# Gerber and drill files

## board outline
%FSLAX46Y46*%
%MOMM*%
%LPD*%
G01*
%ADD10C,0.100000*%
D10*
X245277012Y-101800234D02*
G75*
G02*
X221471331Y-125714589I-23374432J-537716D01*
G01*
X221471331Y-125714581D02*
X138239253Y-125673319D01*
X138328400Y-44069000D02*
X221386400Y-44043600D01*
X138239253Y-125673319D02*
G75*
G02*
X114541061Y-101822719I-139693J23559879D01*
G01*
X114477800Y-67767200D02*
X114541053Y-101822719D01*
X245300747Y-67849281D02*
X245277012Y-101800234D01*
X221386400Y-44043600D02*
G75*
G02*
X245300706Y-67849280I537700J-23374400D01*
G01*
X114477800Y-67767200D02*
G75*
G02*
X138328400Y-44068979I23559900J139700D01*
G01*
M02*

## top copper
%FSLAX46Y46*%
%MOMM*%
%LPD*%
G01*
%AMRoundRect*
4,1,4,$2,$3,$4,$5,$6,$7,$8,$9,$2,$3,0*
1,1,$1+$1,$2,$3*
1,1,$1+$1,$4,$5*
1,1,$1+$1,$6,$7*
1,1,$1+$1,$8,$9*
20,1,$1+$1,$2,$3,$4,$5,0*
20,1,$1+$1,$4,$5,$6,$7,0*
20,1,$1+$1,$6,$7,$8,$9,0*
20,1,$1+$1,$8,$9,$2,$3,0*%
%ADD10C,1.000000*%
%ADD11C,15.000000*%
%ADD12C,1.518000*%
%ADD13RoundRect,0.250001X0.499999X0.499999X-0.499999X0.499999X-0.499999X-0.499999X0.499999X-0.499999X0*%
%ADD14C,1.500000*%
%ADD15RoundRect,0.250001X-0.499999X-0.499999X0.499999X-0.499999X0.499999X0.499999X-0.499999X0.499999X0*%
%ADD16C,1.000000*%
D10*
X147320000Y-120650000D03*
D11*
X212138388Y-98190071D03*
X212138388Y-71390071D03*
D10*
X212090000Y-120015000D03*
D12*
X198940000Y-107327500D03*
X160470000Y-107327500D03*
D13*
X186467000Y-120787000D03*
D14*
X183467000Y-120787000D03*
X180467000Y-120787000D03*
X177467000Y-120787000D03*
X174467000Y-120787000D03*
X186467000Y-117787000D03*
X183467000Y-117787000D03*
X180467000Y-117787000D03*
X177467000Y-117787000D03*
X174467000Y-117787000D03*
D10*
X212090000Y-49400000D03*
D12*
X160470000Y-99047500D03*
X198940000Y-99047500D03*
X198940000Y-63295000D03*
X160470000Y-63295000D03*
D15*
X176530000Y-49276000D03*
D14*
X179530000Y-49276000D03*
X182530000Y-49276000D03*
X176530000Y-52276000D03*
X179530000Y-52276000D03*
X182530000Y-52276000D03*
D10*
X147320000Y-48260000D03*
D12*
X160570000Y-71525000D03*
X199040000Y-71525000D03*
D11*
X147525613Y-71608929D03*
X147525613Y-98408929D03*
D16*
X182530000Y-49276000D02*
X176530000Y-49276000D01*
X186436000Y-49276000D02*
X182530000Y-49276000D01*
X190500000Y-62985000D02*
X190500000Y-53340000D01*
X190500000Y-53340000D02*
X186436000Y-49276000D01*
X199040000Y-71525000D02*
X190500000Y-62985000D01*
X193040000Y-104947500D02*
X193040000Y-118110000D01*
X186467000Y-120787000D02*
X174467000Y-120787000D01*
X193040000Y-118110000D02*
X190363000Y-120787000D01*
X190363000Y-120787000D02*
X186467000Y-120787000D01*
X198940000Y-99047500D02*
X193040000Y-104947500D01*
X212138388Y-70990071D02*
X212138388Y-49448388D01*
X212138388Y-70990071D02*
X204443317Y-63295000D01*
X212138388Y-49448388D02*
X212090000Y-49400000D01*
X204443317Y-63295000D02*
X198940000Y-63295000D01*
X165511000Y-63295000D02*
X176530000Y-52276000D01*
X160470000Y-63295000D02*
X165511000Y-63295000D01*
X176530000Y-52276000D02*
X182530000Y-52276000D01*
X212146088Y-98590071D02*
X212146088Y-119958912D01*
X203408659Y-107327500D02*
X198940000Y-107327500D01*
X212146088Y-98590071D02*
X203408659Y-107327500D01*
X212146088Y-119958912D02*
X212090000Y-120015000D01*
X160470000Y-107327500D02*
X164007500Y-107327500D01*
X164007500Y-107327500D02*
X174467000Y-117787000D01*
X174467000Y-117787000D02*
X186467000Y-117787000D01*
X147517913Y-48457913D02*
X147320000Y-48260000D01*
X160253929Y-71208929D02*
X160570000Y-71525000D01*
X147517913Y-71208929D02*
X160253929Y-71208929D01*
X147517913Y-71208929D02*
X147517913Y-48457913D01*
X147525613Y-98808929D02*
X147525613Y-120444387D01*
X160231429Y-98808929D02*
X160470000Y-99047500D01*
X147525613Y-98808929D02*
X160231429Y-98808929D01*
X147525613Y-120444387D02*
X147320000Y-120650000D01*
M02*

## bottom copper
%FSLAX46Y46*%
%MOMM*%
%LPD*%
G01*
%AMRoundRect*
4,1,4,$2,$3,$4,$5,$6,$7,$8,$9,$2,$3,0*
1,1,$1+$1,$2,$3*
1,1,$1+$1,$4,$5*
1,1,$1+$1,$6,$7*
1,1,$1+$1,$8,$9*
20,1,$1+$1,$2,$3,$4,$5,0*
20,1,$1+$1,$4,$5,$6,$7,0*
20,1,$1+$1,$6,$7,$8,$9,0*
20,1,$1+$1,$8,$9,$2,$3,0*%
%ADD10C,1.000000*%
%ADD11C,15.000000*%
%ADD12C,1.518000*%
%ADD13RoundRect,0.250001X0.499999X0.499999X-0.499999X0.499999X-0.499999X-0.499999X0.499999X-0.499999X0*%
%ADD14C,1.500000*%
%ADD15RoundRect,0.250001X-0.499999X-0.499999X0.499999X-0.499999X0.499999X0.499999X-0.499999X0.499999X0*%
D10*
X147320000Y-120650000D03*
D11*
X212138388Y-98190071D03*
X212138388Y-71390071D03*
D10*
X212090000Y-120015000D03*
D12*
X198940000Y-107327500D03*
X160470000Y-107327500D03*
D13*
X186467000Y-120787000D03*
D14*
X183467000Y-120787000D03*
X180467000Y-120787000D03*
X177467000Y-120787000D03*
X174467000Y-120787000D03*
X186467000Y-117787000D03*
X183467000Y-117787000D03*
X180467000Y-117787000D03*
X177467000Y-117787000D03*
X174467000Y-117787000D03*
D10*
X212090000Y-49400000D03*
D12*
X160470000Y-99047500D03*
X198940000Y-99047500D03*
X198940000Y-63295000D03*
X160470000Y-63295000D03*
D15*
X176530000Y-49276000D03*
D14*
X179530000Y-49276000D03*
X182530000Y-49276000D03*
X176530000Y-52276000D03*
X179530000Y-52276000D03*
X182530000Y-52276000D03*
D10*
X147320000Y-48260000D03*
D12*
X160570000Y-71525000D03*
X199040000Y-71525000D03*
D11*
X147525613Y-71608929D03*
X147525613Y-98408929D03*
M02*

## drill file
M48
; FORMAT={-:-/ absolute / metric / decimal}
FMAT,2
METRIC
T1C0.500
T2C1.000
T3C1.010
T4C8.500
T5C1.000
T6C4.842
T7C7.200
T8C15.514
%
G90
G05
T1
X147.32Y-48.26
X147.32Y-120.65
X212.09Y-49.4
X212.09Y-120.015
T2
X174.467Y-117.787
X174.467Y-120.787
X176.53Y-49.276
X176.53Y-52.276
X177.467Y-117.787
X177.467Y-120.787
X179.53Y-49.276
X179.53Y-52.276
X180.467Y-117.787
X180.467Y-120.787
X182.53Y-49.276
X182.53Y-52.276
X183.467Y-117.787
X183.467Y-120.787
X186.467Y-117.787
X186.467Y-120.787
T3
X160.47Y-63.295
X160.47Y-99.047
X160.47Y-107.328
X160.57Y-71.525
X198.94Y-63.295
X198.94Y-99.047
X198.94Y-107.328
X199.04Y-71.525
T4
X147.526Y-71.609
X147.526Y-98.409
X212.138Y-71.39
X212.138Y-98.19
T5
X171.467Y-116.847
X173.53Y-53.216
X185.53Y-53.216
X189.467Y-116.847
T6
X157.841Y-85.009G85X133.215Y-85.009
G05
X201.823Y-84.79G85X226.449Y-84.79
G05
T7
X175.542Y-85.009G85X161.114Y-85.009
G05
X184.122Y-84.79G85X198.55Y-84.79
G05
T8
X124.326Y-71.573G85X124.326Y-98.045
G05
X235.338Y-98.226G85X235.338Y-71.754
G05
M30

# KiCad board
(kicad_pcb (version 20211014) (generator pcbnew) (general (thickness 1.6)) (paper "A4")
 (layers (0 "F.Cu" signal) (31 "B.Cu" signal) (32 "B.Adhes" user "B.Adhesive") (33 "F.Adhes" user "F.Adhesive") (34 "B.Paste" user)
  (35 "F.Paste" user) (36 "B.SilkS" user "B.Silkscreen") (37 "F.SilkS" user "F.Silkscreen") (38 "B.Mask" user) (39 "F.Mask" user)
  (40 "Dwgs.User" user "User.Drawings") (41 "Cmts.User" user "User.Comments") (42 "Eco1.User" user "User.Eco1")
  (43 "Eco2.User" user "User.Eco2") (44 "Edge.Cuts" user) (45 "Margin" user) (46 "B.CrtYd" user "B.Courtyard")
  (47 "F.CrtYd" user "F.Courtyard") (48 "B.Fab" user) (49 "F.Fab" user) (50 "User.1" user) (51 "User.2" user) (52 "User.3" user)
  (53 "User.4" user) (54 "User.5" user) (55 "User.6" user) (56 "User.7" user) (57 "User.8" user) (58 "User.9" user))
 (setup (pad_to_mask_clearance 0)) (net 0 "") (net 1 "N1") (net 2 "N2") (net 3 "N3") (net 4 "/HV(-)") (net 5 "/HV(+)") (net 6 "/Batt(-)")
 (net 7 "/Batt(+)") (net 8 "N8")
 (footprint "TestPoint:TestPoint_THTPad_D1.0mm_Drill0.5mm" (layer "F.Cu") (at 147.32 120.65)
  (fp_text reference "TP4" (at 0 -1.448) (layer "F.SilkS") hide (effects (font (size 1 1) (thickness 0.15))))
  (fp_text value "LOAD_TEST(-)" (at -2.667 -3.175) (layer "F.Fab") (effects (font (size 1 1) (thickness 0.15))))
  (pad "1" thru_hole circle (at 0 0) (size 1 1) (drill 0.5) (layers *.Cu *.Mask) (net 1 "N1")))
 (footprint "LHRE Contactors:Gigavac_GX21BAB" (layer "F.Cu") (at 182.738388 125.790071 90)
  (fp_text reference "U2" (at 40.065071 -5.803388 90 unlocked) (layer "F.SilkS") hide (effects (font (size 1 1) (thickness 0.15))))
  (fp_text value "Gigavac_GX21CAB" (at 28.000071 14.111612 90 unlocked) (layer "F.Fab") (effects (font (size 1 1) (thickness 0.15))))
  (pad "" np_thru_hole oval (at 41 8.5977 90) (size 7.2 21.6281) (drill oval 7.2 21.6281) (layers F&B.Cu *.Mask))
  (pad "" np_thru_hole oval (at 40.8 52.6 90) (size 41.9862 15.514174) (drill oval 41.9862 15.514174) (layers F&B.Cu *.Mask))
  (pad "" np_thru_hole oval (at 41 31.3977 90) (size 4.84155 29.467172) (drill oval 4.84155 29.467172) (layers F&B.Cu *.Mask))
  (pad "1" thru_hole circle (at 27.6 29.4 90) (size 15 15) (drill 8.5) (layers *.Cu *.Mask) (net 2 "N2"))
  (pad "2" thru_hole circle (at 54.4 29.4 90) (size 15 15) (drill 8.5) (layers *.Cu *.Mask) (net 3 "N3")))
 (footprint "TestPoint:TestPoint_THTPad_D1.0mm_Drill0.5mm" (layer "F.Cu") (at 212.09 120.015)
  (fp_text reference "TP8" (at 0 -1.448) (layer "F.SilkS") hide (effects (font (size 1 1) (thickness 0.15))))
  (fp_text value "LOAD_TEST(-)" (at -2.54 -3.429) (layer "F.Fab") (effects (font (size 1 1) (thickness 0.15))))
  (pad "1" thru_hole circle (at 0 0) (size 1 1) (drill 0.5) (layers *.Cu *.Mask) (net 2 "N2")))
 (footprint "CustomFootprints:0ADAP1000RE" (layer "F.Cu") (at 179.805 114.5175 180)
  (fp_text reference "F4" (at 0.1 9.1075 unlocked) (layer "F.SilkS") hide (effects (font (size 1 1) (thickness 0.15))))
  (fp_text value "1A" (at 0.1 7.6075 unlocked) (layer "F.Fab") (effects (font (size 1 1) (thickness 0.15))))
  (pad "1" thru_hole circle (at -19.135 7.19 180) (size 1.518 1.518) (drill 1.01) (layers *.Cu *.Mask) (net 2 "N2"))
  (pad "2" thru_hole circle (at 19.335 7.19 180) (size 1.518 1.518) (drill 1.01) (layers *.Cu *.Mask) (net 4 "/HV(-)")))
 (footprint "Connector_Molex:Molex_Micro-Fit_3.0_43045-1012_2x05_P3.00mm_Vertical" (layer "F.Cu") (at 186.467 120.787 180)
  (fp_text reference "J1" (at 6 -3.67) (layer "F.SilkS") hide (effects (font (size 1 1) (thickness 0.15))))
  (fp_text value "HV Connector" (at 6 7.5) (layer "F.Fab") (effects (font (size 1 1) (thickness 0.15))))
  (pad "" np_thru_hole circle (at -3 3.94 180) (size 1 1) (drill 1) (layers *.Cu *.Mask))
  (pad "" np_thru_hole circle (at 15 3.94 180) (size 1 1) (drill 1) (layers *.Cu *.Mask))
  (pad "1" thru_hole roundrect (at 0 0 180) (size 1.5 1.5) (drill 1) (layers *.Cu *.Mask) (roundrect_rratio 0.1666673333) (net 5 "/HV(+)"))
  (pad "2" thru_hole circle (at 3 0 180) (size 1.5 1.5) (drill 1) (layers *.Cu *.Mask) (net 5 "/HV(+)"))
  (pad "3" thru_hole circle (at 6 0 180) (size 1.5 1.5) (drill 1) (layers *.Cu *.Mask) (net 5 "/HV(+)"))
  (pad "4" thru_hole circle (at 9 0 180) (size 1.5 1.5) (drill 1) (layers *.Cu *.Mask) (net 5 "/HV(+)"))
  (pad "5" thru_hole circle (at 12 0 180) (size 1.5 1.5) (drill 1) (layers *.Cu *.Mask) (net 5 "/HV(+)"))
  (pad "6" thru_hole circle (at 0 3 180) (size 1.5 1.5) (drill 1) (layers *.Cu *.Mask) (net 4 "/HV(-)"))
  (pad "7" thru_hole circle (at 3 3 180) (size 1.5 1.5) (drill 1) (layers *.Cu *.Mask) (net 4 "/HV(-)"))
  (pad "8" thru_hole circle (at 6 3 180) (size 1.5 1.5) (drill 1) (layers *.Cu *.Mask) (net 4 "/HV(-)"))
  (pad "9" thru_hole circle (at 9 3 180) (size 1.5 1.5) (drill 1) (layers *.Cu *.Mask) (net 4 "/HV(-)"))
  (pad "10" thru_hole circle (at 12 3 180) (size 1.5 1.5) (drill 1) (layers *.Cu *.Mask) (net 4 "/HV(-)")))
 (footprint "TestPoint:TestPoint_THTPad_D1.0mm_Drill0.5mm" (layer "F.Cu") (at 212.09 49.4)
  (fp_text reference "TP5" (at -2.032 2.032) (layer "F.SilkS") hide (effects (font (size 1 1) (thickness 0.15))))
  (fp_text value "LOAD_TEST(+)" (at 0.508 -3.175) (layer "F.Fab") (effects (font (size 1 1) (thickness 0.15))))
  (pad "1" thru_hole circle (at 0 0) (size 1 1) (drill 0.5) (layers *.Cu *.Mask) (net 3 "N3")))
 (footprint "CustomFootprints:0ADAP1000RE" (layer "F.Cu") (at 179.605 91.8575)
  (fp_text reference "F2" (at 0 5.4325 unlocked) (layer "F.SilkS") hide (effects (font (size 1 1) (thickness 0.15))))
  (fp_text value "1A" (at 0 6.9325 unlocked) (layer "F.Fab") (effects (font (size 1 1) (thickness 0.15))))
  (pad "1" thru_hole circle (at -19.135 7.19) (size 1.518 1.518) (drill 1.01) (layers *.Cu *.Mask) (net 1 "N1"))
  (pad "2" thru_hole circle (at 19.335 7.19) (size 1.518 1.518) (drill 1.01) (layers *.Cu *.Mask) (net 5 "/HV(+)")))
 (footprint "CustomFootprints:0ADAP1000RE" (layer "F.Cu") (at 179.805 70.485 180)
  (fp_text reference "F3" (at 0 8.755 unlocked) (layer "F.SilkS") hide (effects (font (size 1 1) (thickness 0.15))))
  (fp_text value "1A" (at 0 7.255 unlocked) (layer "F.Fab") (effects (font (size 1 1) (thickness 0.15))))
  (pad "1" thru_hole circle (at -19.135 7.19 180) (size 1.518 1.518) (drill 1.01) (layers *.Cu *.Mask) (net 3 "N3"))
  (pad "2" thru_hole circle (at 19.335 7.19 180) (size 1.518 1.518) (drill 1.01) (layers *.Cu *.Mask) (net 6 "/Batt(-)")))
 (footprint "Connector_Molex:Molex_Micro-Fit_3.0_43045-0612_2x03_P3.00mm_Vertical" (layer "F.Cu") (at 176.53 49.276)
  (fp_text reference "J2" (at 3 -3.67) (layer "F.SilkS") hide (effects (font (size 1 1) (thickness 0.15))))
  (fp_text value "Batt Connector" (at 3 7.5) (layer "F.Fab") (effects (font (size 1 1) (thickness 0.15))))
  (pad "" np_thru_hole circle (at -3 3.94) (size 1 1) (drill 1) (layers *.Cu *.Mask))
  (pad "" np_thru_hole circle (at 9 3.94) (size 1 1) (drill 1) (layers *.Cu *.Mask))
  (pad "1" thru_hole roundrect (at 0 0) (size 1.5 1.5) (drill 1) (layers *.Cu *.Mask) (roundrect_rratio 0.1666673333) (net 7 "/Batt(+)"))
  (pad "2" thru_hole circle (at 3 0) (size 1.5 1.5) (drill 1) (layers *.Cu *.Mask) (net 7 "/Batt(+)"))
  (pad "3" thru_hole circle (at 6 0) (size 1.5 1.5) (drill 1) (layers *.Cu *.Mask) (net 7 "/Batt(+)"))
  (pad "4" thru_hole circle (at 0 3) (size 1.5 1.5) (drill 1) (layers *.Cu *.Mask) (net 6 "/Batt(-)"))
  (pad "5" thru_hole circle (at 3 3) (size 1.5 1.5) (drill 1) (layers *.Cu *.Mask) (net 6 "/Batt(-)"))
  (pad "6" thru_hole circle (at 6 3) (size 1.5 1.5) (drill 1) (layers *.Cu *.Mask) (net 6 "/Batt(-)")))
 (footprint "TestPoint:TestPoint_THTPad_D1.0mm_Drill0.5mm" (layer "F.Cu") (at 147.32 48.26)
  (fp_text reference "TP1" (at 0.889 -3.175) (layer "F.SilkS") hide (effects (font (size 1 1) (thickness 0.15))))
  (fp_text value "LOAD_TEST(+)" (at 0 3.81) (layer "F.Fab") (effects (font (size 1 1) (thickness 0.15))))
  (pad "1" thru_hole circle (at 0 0) (size 1 1) (drill 0.5) (layers *.Cu *.Mask) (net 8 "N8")))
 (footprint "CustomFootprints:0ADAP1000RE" (layer "F.Cu") (at 179.705 64.335)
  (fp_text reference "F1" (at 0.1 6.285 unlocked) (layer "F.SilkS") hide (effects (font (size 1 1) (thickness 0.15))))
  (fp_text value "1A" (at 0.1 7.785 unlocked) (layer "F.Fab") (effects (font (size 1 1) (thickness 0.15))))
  (pad "1" thru_hole circle (at -19.135 7.19) (size 1.518 1.518) (drill 1.01) (layers *.Cu *.Mask) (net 8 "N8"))
  (pad "2" thru_hole circle (at 19.335 7.19) (size 1.518 1.518) (drill 1.01) (layers *.Cu *.Mask) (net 7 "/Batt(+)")))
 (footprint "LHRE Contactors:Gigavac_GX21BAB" (layer "F.Cu") (at 176.925613 44.008929 -90)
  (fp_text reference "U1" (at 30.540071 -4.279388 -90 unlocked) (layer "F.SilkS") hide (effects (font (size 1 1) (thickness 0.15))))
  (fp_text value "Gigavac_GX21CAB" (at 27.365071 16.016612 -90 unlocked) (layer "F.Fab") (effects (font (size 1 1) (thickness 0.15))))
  (pad "" np_thru_hole oval (at 40.8 52.6 270) (size 41.9862 15.514174) (drill oval 41.9862 15.514174) (layers F&B.Cu *.Mask))
  (pad "" np_thru_hole oval (at 41 31.3977 270) (size 4.84155 29.467172) (drill oval 4.84155 29.467172) (layers F&B.Cu *.Mask))
  (pad "" np_thru_hole oval (at 41 8.5977 270) (size 7.2 21.6281) (drill oval 7.2 21.6281) (layers F&B.Cu *.Mask))
  (pad "1" thru_hole circle (at 27.6 29.4 270) (size 15 15) (drill 8.5) (layers *.Cu *.Mask) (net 8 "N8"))
  (pad "2" thru_hole circle (at 54.4 29.4 270) (size 15 15) (drill 8.5) (layers *.Cu *.Mask) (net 1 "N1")))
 (gr_arc (start 245.277012 101.800234) (mid 238.472778 118.832846) (end 221.471331 125.714581) (layer "Edge.Cuts") (width 0.1))
 (gr_line (start 221.471331 125.714581) (end 138.239253 125.673319) (layer "Edge.Cuts") (width 0.1))
 (gr_line (start 138.3284 44.069) (end 221.3864 44.0436) (layer "Edge.Cuts") (width 0.1))
 (gr_arc (start 138.239253 125.673319) (mid 121.3866 118.7196) (end 114.541053 101.822719) (layer "Edge.Cuts") (width 0.1))
 (gr_line (start 114.4778 67.7672) (end 114.541053 101.822719) (layer "Edge.Cuts") (width 0.1))
 (gr_line (start 245.300747 67.849281) (end 245.277012 101.800234) (layer "Edge.Cuts") (width 0.1))
 (gr_arc (start 221.3864 44.0436) (mid 238.419012 50.847834) (end 245.300747 67.849281) (layer "Edge.Cuts") (width 0.1))
 (gr_arc (start 114.4778 67.7672) (mid 121.431519 50.914547) (end 138.3284 44.069) (layer "Edge.Cuts") (width 0.1))
 (segment (start 182.53 49.276) (end 176.53 49.276) (width 1) (layer "F.Cu") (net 7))
 (segment (start 186.436 49.276) (end 182.53 49.276) (width 1) (layer "F.Cu") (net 7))
 (segment (start 190.5 62.985) (end 190.5 53.34) (width 1) (layer "F.Cu") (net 7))
 (segment (start 190.5 53.34) (end 186.436 49.276) (width 1) (layer "F.Cu") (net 7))
 (segment (start 199.04 71.525) (end 190.5 62.985) (width 1) (layer "F.Cu") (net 7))
 (segment (start 193.04 104.9475) (end 193.04 118.11) (width 1) (layer "F.Cu") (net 5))
 (segment (start 186.467 120.787) (end 174.467 120.787) (width 1) (layer "F.Cu") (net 5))
 (segment (start 193.04 118.11) (end 190.363 120.787) (width 1) (layer "F.Cu") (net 5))
 (segment (start 190.363 120.787) (end 186.467 120.787) (width 1) (layer "F.Cu") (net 5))
 (segment (start 198.94 99.0475) (end 193.04 104.9475) (width 1) (layer "F.Cu") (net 5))
 (segment (start 212.138388 70.990071) (end 212.138388 49.448388) (width 1) (layer "F.Cu") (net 3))
 (segment (start 212.138388 70.990071) (end 204.443317 63.295) (width 1) (layer "F.Cu") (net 3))
 (segment (start 212.138388 49.448388) (end 212.09 49.4) (width 1) (layer "F.Cu") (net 3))
 (segment (start 204.443317 63.295) (end 198.94 63.295) (width 1) (layer "F.Cu") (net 3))
 (segment (start 165.511 63.295) (end 176.53 52.276) (width 1) (layer "F.Cu") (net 6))
 (segment (start 160.47 63.295) (end 165.511 63.295) (width 1) (layer "F.Cu") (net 6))
 (segment (start 176.53 52.276) (end 182.53 52.276) (width 1) (layer "F.Cu") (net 6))
 (segment (start 212.146088 98.590071) (end 212.146088 119.958912) (width 1) (layer "F.Cu") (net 2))
 (segment (start 203.408659 107.3275) (end 198.94 107.3275) (width 1) (layer "F.Cu") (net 2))
 (segment (start 212.146088 98.590071) (end 203.408659 107.3275) (width 1) (layer "F.Cu") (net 2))
 (segment (start 212.146088 119.958912) (end 212.09 120.015) (width 1) (layer "F.Cu") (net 2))
 (segment (start 160.47 107.3275) (end 164.0075 107.3275) (width 1) (layer "F.Cu") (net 4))
 (segment (start 164.0075 107.3275) (end 174.467 117.787) (width 1) (layer "F.Cu") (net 4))
 (segment (start 174.467 117.787) (end 186.467 117.787) (width 1) (layer "F.Cu") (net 4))
 (segment (start 147.517913 48.457913) (end 147.32 48.26) (width 1) (layer "F.Cu") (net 8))
 (segment (start 160.253929 71.208929) (end 160.57 71.525) (width 1) (layer "F.Cu") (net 8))
 (segment (start 147.517913 71.208929) (end 160.253929 71.208929) (width 1) (layer "F.Cu") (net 8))
 (segment (start 147.517913 71.208929) (end 147.517913 48.457913) (width 1) (layer "F.Cu") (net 8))
 (segment (start 147.525613 98.808929) (end 147.525613 120.444387) (width 1) (layer "F.Cu") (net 1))
 (segment (start 160.231429 98.808929) (end 160.47 99.0475) (width 1) (layer "F.Cu") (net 1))
 (segment (start 147.525613 98.808929) (end 160.231429 98.808929) (width 1) (layer "F.Cu") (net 1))
 (segment (start 147.525613 120.444387) (end 147.32 120.65) (width 1) (layer "F.Cu") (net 1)))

